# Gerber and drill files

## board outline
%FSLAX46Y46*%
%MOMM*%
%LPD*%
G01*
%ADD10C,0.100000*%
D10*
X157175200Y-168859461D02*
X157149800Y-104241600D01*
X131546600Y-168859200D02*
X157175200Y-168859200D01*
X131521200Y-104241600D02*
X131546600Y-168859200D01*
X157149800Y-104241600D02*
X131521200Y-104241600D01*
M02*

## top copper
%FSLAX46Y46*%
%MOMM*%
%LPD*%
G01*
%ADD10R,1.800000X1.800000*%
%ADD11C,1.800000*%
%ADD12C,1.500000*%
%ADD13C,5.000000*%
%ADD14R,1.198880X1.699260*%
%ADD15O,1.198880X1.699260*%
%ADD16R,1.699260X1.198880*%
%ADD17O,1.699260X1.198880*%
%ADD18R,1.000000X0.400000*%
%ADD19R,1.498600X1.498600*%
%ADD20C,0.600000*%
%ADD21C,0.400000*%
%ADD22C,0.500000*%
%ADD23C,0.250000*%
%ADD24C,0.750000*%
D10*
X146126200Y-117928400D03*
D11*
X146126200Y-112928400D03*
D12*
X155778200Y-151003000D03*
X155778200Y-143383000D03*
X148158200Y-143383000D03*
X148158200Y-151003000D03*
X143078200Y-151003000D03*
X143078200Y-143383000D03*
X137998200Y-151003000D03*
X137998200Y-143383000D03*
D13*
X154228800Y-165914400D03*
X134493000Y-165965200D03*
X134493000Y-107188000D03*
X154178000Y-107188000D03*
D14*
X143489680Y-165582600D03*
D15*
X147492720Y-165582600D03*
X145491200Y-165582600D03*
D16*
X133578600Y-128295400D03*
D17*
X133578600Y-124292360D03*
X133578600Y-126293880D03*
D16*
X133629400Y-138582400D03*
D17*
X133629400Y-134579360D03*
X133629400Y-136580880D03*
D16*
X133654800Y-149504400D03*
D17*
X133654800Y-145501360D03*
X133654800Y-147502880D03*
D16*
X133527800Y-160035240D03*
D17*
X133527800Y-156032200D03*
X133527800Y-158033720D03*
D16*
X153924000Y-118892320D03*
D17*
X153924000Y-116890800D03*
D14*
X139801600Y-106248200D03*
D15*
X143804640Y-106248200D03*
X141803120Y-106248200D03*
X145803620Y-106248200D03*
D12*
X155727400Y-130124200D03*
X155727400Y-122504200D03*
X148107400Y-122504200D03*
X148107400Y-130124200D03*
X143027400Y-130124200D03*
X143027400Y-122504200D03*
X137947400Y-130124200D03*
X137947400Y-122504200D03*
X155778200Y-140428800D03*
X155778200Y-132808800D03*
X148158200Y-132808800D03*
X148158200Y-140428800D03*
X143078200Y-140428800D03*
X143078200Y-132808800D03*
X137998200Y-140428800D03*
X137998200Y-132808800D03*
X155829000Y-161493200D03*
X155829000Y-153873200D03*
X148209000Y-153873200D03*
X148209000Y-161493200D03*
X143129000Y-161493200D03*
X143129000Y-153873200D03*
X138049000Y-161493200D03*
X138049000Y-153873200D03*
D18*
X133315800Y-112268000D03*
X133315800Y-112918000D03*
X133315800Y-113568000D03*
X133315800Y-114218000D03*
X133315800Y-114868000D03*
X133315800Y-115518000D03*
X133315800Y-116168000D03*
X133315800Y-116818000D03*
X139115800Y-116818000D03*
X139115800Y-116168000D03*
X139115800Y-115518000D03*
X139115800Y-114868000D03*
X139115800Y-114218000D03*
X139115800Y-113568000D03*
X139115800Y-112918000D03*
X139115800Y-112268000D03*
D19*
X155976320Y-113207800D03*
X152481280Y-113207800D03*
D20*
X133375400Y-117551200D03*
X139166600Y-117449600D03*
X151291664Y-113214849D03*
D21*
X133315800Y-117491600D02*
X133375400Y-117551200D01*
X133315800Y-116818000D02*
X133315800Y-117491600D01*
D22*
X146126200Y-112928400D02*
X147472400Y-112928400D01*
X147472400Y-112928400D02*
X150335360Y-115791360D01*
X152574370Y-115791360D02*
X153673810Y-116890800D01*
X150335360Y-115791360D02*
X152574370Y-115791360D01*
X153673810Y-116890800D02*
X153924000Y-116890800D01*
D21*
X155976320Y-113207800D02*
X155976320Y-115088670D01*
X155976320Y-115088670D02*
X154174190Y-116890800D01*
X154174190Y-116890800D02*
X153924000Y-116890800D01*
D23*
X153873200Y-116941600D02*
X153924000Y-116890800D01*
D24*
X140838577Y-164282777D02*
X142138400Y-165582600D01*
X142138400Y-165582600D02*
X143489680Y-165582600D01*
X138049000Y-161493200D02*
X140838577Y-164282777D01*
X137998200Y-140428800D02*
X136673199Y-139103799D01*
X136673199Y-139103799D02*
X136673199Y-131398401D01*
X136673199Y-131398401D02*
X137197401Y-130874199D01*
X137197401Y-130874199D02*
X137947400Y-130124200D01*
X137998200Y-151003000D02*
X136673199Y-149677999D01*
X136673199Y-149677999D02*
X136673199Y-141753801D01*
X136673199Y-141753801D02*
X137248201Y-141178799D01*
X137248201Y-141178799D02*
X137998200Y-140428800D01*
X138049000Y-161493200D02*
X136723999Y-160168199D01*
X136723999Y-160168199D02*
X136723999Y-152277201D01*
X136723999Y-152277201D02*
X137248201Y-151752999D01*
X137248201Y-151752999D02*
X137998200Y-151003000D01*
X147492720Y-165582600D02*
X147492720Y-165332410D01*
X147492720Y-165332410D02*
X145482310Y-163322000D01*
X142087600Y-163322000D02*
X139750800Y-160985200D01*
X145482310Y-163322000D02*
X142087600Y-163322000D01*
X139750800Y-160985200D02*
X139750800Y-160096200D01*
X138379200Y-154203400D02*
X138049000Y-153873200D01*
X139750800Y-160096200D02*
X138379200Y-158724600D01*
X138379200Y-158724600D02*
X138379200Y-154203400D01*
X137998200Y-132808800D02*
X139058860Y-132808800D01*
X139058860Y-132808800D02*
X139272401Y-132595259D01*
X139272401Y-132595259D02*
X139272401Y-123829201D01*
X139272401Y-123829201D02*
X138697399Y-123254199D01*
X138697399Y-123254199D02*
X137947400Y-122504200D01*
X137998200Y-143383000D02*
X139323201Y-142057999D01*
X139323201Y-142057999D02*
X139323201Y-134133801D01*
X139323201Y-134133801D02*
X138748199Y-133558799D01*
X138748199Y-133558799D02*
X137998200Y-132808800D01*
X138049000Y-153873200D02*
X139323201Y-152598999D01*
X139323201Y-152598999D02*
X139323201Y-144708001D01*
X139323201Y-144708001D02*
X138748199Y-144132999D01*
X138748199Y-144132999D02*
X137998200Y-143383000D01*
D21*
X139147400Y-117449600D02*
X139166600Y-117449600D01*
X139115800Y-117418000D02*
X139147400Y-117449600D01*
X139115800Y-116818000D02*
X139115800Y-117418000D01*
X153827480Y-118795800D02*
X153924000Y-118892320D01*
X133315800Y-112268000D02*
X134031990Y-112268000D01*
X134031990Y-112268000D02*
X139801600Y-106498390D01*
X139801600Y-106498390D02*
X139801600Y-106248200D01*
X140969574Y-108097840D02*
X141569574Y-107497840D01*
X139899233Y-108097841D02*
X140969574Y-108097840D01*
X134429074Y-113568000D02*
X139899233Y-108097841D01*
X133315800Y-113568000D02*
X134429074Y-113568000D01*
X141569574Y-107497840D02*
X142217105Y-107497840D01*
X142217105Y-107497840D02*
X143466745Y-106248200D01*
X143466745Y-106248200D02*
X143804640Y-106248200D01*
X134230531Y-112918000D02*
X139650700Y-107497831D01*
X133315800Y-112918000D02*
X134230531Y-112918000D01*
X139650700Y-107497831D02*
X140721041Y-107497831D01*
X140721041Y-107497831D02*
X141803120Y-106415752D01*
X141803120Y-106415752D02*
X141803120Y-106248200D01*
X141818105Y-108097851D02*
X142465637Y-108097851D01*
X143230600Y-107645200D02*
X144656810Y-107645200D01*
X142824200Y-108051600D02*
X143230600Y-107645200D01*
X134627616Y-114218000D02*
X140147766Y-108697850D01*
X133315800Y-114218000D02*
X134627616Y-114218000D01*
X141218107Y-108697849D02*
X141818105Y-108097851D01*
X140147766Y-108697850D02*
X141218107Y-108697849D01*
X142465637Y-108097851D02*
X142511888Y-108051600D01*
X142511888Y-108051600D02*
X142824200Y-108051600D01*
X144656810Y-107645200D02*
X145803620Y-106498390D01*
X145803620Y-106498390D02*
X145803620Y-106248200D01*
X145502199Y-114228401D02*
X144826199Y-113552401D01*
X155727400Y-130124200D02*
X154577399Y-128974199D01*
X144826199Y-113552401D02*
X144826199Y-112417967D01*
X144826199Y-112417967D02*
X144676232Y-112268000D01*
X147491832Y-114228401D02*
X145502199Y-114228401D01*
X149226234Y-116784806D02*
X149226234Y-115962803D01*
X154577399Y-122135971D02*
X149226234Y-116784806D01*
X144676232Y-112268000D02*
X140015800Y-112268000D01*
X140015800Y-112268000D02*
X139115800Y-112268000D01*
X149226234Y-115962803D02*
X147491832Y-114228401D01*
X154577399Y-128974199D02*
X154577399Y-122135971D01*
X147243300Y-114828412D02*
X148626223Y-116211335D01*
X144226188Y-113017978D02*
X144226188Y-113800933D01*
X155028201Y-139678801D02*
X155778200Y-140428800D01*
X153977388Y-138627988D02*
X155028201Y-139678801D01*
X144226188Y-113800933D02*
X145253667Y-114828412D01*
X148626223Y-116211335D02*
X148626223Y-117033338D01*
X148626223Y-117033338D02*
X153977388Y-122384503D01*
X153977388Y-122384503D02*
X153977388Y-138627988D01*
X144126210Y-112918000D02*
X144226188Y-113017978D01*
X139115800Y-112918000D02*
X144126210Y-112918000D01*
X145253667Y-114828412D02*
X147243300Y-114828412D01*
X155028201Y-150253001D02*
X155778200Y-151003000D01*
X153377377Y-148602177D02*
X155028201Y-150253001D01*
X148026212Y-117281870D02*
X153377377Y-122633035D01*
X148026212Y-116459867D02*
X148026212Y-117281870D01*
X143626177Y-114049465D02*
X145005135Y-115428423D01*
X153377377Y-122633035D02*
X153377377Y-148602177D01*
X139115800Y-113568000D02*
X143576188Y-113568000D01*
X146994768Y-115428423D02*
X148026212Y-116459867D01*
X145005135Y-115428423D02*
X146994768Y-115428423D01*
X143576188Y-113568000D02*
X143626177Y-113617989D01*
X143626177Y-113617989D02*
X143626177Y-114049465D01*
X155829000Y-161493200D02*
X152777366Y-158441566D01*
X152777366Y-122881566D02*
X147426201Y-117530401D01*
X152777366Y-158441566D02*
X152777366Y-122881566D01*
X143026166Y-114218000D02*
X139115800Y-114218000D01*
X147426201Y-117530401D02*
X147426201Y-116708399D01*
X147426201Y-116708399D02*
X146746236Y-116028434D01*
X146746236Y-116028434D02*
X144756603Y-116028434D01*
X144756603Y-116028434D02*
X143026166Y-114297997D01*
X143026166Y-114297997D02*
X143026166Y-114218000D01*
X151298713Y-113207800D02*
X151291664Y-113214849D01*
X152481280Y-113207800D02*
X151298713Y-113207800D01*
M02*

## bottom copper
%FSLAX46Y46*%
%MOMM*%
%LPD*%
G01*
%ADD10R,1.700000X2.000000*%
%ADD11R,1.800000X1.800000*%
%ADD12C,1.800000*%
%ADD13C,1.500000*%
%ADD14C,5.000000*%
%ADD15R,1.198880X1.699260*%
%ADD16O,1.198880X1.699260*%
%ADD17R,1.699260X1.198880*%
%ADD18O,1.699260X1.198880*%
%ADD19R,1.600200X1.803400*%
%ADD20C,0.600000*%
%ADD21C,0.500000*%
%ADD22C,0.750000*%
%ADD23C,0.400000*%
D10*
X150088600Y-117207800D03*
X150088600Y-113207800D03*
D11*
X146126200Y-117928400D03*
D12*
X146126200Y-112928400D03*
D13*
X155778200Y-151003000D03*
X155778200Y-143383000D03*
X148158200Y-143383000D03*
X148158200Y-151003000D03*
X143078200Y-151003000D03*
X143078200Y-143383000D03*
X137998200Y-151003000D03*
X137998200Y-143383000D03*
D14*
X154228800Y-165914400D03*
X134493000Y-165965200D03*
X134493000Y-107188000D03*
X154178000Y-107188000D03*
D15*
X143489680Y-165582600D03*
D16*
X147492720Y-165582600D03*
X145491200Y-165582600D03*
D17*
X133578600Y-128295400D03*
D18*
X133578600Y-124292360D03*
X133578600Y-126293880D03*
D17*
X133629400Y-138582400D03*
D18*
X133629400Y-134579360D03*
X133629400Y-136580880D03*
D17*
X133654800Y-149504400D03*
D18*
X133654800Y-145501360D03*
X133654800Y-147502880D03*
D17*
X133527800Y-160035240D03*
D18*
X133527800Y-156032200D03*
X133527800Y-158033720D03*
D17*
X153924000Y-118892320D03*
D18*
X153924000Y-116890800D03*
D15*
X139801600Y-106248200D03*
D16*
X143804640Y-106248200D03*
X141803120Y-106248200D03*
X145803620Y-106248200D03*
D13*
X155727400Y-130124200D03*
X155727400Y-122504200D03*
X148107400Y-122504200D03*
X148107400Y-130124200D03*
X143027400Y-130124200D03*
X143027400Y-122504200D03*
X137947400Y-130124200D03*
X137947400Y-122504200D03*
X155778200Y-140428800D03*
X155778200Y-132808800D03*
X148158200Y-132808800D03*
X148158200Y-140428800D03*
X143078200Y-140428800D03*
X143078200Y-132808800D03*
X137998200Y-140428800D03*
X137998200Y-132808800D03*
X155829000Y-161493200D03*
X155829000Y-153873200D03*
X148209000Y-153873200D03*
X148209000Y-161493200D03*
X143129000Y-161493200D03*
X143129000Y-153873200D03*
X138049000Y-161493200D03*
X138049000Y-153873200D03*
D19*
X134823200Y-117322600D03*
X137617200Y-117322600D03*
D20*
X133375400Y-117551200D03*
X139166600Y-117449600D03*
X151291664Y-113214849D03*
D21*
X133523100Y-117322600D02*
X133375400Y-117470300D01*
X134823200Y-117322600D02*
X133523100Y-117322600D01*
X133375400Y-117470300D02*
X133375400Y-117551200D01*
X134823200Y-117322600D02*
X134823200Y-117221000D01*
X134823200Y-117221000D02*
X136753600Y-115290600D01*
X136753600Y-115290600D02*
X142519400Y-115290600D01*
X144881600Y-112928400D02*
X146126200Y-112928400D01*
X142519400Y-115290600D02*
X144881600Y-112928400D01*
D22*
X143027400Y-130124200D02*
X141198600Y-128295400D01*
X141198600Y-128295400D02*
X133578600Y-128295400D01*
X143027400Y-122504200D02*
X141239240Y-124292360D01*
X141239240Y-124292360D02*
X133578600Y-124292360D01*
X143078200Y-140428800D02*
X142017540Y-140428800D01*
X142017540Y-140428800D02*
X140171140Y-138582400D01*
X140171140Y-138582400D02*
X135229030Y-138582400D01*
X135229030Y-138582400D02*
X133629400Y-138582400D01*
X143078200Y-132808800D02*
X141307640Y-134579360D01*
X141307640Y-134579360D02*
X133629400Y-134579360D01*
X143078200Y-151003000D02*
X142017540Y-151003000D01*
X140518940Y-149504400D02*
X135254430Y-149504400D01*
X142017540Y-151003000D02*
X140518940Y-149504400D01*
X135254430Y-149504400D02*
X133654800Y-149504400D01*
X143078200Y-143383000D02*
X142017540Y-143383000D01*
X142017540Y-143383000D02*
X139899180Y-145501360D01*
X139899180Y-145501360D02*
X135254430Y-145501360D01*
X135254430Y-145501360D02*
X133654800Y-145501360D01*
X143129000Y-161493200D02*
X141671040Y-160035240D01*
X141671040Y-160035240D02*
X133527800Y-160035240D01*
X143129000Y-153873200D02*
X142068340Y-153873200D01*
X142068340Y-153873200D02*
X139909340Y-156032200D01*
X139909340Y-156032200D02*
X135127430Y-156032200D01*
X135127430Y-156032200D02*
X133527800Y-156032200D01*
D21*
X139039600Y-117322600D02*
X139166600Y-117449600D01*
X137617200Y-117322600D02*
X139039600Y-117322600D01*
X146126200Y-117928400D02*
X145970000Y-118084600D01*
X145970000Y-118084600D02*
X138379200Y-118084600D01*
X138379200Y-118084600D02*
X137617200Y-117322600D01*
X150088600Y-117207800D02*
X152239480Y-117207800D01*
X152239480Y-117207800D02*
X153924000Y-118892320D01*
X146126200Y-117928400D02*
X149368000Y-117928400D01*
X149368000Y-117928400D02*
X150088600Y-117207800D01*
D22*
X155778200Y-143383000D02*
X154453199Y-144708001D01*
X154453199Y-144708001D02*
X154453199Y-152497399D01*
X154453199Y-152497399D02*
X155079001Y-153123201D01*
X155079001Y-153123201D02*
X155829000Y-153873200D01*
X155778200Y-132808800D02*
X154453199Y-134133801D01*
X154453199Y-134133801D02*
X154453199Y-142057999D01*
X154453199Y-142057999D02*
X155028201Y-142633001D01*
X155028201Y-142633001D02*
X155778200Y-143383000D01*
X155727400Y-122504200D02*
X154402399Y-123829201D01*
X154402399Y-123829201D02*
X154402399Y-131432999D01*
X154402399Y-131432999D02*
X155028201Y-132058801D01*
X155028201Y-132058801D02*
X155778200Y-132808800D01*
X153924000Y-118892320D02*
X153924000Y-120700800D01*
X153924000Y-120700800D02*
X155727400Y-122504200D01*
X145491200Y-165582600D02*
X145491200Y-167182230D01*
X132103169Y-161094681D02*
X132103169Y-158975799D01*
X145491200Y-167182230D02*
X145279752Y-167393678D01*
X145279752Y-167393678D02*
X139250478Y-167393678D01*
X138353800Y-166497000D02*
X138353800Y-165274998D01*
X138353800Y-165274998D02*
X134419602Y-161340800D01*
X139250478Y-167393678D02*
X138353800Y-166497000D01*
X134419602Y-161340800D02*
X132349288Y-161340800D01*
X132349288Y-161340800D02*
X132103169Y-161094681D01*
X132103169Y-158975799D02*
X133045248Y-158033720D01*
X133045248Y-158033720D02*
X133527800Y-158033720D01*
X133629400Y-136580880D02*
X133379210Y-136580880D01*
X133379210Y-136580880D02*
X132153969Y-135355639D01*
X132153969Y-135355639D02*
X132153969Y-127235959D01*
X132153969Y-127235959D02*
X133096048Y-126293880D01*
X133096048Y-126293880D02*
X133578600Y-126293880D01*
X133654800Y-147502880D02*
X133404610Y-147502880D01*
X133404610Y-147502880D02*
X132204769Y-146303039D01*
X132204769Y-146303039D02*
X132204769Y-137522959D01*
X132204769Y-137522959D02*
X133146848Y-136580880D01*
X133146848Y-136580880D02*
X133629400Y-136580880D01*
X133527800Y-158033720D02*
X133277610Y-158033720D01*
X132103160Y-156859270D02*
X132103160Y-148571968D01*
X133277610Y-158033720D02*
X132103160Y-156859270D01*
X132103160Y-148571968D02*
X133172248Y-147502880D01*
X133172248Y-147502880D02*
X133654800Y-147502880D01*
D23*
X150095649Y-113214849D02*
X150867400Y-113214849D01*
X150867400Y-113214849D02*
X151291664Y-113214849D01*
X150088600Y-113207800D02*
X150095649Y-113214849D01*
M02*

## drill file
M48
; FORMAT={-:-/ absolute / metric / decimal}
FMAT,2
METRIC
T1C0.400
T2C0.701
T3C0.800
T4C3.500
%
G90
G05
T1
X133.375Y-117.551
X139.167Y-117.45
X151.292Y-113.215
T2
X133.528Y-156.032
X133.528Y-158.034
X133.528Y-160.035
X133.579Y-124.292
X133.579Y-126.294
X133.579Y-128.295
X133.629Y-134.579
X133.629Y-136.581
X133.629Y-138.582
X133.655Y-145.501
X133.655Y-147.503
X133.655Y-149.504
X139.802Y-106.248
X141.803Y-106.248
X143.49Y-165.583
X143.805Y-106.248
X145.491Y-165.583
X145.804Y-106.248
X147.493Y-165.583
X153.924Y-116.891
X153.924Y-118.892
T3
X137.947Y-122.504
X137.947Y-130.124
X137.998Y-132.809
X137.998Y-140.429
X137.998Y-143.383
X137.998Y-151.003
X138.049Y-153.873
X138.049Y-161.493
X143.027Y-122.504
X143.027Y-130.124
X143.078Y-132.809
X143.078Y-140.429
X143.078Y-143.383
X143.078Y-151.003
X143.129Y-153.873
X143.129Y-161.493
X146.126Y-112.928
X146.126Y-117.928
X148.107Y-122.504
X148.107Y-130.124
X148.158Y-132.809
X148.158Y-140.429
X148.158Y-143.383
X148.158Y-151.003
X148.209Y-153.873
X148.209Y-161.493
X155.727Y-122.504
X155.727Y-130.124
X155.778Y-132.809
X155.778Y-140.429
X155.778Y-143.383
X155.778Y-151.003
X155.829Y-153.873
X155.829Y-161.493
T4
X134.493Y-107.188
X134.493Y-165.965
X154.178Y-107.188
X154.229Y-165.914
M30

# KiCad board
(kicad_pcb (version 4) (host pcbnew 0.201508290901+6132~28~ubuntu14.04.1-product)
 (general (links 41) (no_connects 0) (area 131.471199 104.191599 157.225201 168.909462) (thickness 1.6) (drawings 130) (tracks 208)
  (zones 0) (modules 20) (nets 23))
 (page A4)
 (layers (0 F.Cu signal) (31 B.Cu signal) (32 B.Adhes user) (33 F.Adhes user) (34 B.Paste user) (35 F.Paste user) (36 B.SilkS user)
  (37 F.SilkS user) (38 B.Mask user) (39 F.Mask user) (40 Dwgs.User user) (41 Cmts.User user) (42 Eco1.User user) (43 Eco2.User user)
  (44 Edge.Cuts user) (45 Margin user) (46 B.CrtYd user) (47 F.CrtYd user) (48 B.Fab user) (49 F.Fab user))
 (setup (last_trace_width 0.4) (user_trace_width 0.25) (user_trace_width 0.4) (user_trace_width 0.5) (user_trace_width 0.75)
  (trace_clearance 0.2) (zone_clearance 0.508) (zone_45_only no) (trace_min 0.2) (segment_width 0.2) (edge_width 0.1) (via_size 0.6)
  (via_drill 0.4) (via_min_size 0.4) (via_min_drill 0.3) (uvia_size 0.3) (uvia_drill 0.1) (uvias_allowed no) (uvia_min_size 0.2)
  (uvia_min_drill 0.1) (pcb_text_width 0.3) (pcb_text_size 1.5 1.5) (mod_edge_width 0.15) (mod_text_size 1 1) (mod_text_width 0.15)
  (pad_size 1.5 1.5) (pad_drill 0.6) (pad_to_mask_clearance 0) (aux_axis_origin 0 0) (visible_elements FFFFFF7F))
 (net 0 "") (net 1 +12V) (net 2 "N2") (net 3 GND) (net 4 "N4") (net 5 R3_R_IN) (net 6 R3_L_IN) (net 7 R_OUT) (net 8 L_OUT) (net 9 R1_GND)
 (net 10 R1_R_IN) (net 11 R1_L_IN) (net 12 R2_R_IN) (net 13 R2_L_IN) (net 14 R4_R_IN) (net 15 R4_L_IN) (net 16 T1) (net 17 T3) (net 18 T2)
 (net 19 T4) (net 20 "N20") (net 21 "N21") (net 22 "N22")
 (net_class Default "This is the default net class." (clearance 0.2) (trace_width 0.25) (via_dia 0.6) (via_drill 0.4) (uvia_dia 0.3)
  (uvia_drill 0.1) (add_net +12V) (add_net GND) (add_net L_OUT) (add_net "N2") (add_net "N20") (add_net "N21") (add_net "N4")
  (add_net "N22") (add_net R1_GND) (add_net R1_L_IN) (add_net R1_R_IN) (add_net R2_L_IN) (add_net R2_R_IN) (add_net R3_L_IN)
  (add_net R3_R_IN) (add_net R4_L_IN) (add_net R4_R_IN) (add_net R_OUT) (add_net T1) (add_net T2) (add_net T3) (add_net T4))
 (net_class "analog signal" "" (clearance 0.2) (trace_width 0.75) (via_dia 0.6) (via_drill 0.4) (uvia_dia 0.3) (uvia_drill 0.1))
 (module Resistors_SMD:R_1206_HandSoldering (layer B.Cu) (at 150.0886 115.2078 90)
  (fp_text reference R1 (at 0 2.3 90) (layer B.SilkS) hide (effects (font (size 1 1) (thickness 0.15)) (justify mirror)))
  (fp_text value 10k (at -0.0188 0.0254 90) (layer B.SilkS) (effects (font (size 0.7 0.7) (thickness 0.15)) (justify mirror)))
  (pad 1 smd rect (at -2 0 90) (size 2 1.7) (layers B.Cu B.Paste B.Mask) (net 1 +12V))
  (pad 2 smd rect (at 2 0 90) (size 2 1.7) (layers B.Cu B.Paste B.Mask) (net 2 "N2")))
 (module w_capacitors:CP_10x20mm (layer F.Cu) (at 146.1262 115.4284)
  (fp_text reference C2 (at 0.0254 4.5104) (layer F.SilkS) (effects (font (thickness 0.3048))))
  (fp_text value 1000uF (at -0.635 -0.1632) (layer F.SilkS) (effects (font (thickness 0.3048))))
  (pad 1 thru_hole rect (at 0 2.5) (size 1.8 1.8) (drill 0.8) (layers *.Cu *.Mask F.SilkS) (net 1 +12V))
  (pad 2 thru_hole circle (at 0 -2.5) (size 1.8 1.8) (drill 0.8) (layers *.Cu *.Mask F.SilkS) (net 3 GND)))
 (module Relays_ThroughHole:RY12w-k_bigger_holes (layer F.Cu) (at 156.9782 152.103 180)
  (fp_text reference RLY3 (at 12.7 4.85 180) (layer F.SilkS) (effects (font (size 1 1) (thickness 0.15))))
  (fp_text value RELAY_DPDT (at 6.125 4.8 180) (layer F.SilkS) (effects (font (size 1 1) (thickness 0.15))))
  (pad 1 thru_hole circle (at 1.2 1.1 180) (size 1.5 1.5) (drill 0.8) (layers *.Cu *.Mask F.SilkS) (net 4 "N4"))
  (pad 8 thru_hole circle (at 1.2 8.72 180) (size 1.5 1.5) (drill 0.8) (layers *.Cu *.Mask F.SilkS) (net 1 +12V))
  (pad 7 thru_hole circle (at 8.82 8.72 180) (size 1.5 1.5) (drill 0.8) (layers *.Cu *.Mask F.SilkS))
  (pad 2 thru_hole circle (at 8.82 1.1 180) (size 1.5 1.5) (drill 0.8) (layers *.Cu *.Mask F.SilkS))
  (pad 3 thru_hole circle (at 13.9 1.1 180) (size 1.5 1.5) (drill 0.8) (layers *.Cu *.Mask F.SilkS) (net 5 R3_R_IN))
  (pad 6 thru_hole circle (at 13.9 8.72 180) (size 1.5 1.5) (drill 0.8) (layers *.Cu *.Mask F.SilkS) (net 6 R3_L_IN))
  (pad 4 thru_hole circle (at 18.98 1.1 180) (size 1.5 1.5) (drill 0.8) (layers *.Cu *.Mask F.SilkS) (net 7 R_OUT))
  (pad 5 thru_hole circle (at 18.98 8.72 180) (size 1.5 1.5) (drill 0.8) (layers *.Cu *.Mask F.SilkS) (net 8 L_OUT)))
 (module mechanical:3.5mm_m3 (layer F.Cu) (at 154.2288 166.0144)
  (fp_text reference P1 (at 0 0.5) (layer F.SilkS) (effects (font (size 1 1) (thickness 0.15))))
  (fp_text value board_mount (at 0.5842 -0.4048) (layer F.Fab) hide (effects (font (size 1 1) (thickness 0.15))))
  (pad 1 thru_hole circle (at 0 -0.1) (size 5 5) (drill 3.5) (layers *.Cu *.Mask F.SilkS)))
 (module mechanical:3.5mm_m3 (layer F.Cu) (at 134.493 166.0652)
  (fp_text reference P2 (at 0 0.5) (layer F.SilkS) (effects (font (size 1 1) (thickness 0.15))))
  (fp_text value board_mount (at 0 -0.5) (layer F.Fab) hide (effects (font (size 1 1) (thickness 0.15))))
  (pad 1 thru_hole circle (at 0 -0.1) (size 5 5) (drill 3.5) (layers *.Cu *.Mask F.SilkS)))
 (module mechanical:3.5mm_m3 (layer F.Cu) (at 134.493 107.288)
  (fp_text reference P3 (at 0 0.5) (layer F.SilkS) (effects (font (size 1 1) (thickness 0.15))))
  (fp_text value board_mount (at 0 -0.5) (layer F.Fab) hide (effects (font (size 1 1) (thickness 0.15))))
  (pad 1 thru_hole circle (at 0 -0.1) (size 5 5) (drill 3.5) (layers *.Cu *.Mask F.SilkS)))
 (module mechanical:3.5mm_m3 (layer F.Cu) (at 154.178 107.288)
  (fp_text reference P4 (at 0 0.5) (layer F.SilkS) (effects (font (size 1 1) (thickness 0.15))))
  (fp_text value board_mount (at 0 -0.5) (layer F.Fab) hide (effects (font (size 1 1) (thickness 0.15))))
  (pad 1 thru_hole circle (at 0 -0.1) (size 5 5) (drill 3.5) (layers *.Cu *.Mask F.SilkS)))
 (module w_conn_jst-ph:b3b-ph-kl (layer F.Cu) (at 145.4912 165.5826)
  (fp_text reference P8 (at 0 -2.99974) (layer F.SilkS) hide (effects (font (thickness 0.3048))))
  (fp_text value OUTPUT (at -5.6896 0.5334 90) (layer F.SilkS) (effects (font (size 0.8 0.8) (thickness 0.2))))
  (pad 1 thru_hole rect (at -2.00152 0) (size 1.19888 1.69926) (drill 0.70104) (layers *.Cu *.Mask F.SilkS) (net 7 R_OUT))
  (pad 3 thru_hole oval (at 2.00152 0) (size 1.19888 1.69926) (drill 0.70104) (layers *.Cu *.Mask F.SilkS) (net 8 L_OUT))
  (pad 2 thru_hole oval (at 0 0) (size 1.19888 1.69926) (drill 0.70104) (layers *.Cu *.Mask F.SilkS) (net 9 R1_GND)))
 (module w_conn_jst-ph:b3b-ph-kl (layer F.Cu) (at 133.5786 126.29388 90)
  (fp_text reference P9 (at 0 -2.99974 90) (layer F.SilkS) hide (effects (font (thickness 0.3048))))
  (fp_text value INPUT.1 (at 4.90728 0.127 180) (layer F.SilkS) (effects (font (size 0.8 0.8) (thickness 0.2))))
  (pad 1 thru_hole rect (at -2.00152 0 90) (size 1.19888 1.69926) (drill 0.70104) (layers *.Cu *.Mask F.SilkS) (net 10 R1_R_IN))
  (pad 3 thru_hole oval (at 2.00152 0 90) (size 1.19888 1.69926) (drill 0.70104) (layers *.Cu *.Mask F.SilkS) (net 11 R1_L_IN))
  (pad 2 thru_hole oval (at 0 0 90) (size 1.19888 1.69926) (drill 0.70104) (layers *.Cu *.Mask F.SilkS) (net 9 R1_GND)))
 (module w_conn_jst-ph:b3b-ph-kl (layer F.Cu) (at 133.6294 136.58088 90)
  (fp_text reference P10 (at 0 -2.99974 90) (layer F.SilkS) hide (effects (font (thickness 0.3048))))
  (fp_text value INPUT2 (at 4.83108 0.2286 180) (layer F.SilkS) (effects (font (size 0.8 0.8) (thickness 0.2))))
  (pad 1 thru_hole rect (at -2.00152 0 90) (size 1.19888 1.69926) (drill 0.70104) (layers *.Cu *.Mask F.SilkS) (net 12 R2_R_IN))
  (pad 3 thru_hole oval (at 2.00152 0 90) (size 1.19888 1.69926) (drill 0.70104) (layers *.Cu *.Mask F.SilkS) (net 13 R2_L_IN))
  (pad 2 thru_hole oval (at 0 0 90) (size 1.19888 1.69926) (drill 0.70104) (layers *.Cu *.Mask F.SilkS) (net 9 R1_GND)))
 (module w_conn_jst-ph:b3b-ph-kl (layer F.Cu) (at 133.6548 147.50288 90)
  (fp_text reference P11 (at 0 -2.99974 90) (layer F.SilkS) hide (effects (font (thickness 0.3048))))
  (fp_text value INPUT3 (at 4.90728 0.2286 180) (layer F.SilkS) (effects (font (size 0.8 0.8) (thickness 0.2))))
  (pad 1 thru_hole rect (at -2.00152 0 90) (size 1.19888 1.69926) (drill 0.70104) (layers *.Cu *.Mask F.SilkS) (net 5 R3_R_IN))
  (pad 3 thru_hole oval (at 2.00152 0 90) (size 1.19888 1.69926) (drill 0.70104) (layers *.Cu *.Mask F.SilkS) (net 6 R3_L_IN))
  (pad 2 thru_hole oval (at 0 0 90) (size 1.19888 1.69926) (drill 0.70104) (layers *.Cu *.Mask F.SilkS) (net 9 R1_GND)))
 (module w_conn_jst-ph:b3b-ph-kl (layer F.Cu) (at 133.5278 158.03372 90)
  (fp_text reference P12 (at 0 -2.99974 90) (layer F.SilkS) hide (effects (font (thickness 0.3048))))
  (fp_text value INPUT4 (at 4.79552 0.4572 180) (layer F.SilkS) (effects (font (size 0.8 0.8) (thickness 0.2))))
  (pad 1 thru_hole rect (at -2.00152 0 90) (size 1.19888 1.69926) (drill 0.70104) (layers *.Cu *.Mask F.SilkS) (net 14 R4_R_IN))
  (pad 3 thru_hole oval (at 2.00152 0 90) (size 1.19888 1.69926) (drill 0.70104) (layers *.Cu *.Mask F.SilkS) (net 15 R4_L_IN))
  (pad 2 thru_hole oval (at 0 0 90) (size 1.19888 1.69926) (drill 0.70104) (layers *.Cu *.Mask F.SilkS) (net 9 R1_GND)))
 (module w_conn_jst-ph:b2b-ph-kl (layer F.Cu) (at 153.924 117.89156 90)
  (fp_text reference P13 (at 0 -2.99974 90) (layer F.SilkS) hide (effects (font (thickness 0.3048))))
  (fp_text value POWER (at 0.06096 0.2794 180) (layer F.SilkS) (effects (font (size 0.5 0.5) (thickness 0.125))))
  (pad 1 thru_hole rect (at -1.00076 0 90) (size 1.19888 1.69926) (drill 0.70104) (layers *.Cu *.Mask F.SilkS) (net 1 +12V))
  (pad 2 thru_hole oval (at 1.00076 0 90) (size 1.19888 1.69926) (drill 0.70104) (layers *.Cu *.Mask F.SilkS) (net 3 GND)))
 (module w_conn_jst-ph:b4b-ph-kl (layer F.Cu) (at 142.80388 106.2482)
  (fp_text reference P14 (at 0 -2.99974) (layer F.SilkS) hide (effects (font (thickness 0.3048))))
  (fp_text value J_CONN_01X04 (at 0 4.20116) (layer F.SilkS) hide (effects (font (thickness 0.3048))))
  (pad 1 thru_hole rect (at -3.00228 0) (size 1.19888 1.69926) (drill 0.70104) (layers *.Cu *.Mask F.SilkS) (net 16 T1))
  (pad 3 thru_hole oval (at 1.00076 0) (size 1.19888 1.69926) (drill 0.70104) (layers *.Cu *.Mask F.SilkS) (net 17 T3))
  (pad 2 thru_hole oval (at -1.00076 0) (size 1.19888 1.69926) (drill 0.70104) (layers *.Cu *.Mask F.SilkS) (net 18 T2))
  (pad 4 thru_hole oval (at 2.99974 0) (size 1.19888 1.69926) (drill 0.70104) (layers *.Cu *.Mask F.SilkS) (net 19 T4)))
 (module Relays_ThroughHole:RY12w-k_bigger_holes (layer F.Cu) (at 156.9274 131.2242 180)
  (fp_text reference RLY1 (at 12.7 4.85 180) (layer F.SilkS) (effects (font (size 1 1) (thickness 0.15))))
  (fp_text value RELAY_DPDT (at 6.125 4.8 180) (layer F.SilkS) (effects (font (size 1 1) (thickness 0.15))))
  (pad 1 thru_hole circle (at 1.2 1.1 180) (size 1.5 1.5) (drill 0.8) (layers *.Cu *.Mask F.SilkS) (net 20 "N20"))
  (pad 8 thru_hole circle (at 1.2 8.72 180) (size 1.5 1.5) (drill 0.8) (layers *.Cu *.Mask F.SilkS) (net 1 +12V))
  (pad 7 thru_hole circle (at 8.82 8.72 180) (size 1.5 1.5) (drill 0.8) (layers *.Cu *.Mask F.SilkS))
  (pad 2 thru_hole circle (at 8.82 1.1 180) (size 1.5 1.5) (drill 0.8) (layers *.Cu *.Mask F.SilkS))
  (pad 3 thru_hole circle (at 13.9 1.1 180) (size 1.5 1.5) (drill 0.8) (layers *.Cu *.Mask F.SilkS) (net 10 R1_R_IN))
  (pad 6 thru_hole circle (at 13.9 8.72 180) (size 1.5 1.5) (drill 0.8) (layers *.Cu *.Mask F.SilkS) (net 11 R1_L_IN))
  (pad 4 thru_hole circle (at 18.98 1.1 180) (size 1.5 1.5) (drill 0.8) (layers *.Cu *.Mask F.SilkS) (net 7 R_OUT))
  (pad 5 thru_hole circle (at 18.98 8.72 180) (size 1.5 1.5) (drill 0.8) (layers *.Cu *.Mask F.SilkS) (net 8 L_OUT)))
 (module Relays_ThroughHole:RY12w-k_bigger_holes (layer F.Cu) (at 156.9782 141.5288 180)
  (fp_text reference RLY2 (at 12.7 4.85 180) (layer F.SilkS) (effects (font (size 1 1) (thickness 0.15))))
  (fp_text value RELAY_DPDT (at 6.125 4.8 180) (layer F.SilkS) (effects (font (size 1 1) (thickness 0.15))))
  (pad 1 thru_hole circle (at 1.2 1.1 180) (size 1.5 1.5) (drill 0.8) (layers *.Cu *.Mask F.SilkS) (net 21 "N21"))
  (pad 8 thru_hole circle (at 1.2 8.72 180) (size 1.5 1.5) (drill 0.8) (layers *.Cu *.Mask F.SilkS) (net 1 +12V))
  (pad 7 thru_hole circle (at 8.82 8.72 180) (size 1.5 1.5) (drill 0.8) (layers *.Cu *.Mask F.SilkS))
  (pad 2 thru_hole circle (at 8.82 1.1 180) (size 1.5 1.5) (drill 0.8) (layers *.Cu *.Mask F.SilkS))
  (pad 3 thru_hole circle (at 13.9 1.1 180) (size 1.5 1.5) (drill 0.8) (layers *.Cu *.Mask F.SilkS) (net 12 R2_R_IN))
  (pad 6 thru_hole circle (at 13.9 8.72 180) (size 1.5 1.5) (drill 0.8) (layers *.Cu *.Mask F.SilkS) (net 13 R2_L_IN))
  (pad 4 thru_hole circle (at 18.98 1.1 180) (size 1.5 1.5) (drill 0.8) (layers *.Cu *.Mask F.SilkS) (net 7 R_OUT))
  (pad 5 thru_hole circle (at 18.98 8.72 180) (size 1.5 1.5) (drill 0.8) (layers *.Cu *.Mask F.SilkS) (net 8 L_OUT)))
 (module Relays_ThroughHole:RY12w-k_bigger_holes (layer F.Cu) (at 157.029 162.5932 180)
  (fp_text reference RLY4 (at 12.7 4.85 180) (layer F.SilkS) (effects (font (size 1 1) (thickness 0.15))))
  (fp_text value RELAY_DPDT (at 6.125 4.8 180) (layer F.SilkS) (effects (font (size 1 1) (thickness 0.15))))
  (pad 1 thru_hole circle (at 1.2 1.1 180) (size 1.5 1.5) (drill 0.8) (layers *.Cu *.Mask F.SilkS) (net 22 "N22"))
  (pad 8 thru_hole circle (at 1.2 8.72 180) (size 1.5 1.5) (drill 0.8) (layers *.Cu *.Mask F.SilkS) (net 1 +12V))
  (pad 7 thru_hole circle (at 8.82 8.72 180) (size 1.5 1.5) (drill 0.8) (layers *.Cu *.Mask F.SilkS))
  (pad 2 thru_hole circle (at 8.82 1.1 180) (size 1.5 1.5) (drill 0.8) (layers *.Cu *.Mask F.SilkS))
  (pad 3 thru_hole circle (at 13.9 1.1 180) (size 1.5 1.5) (drill 0.8) (layers *.Cu *.Mask F.SilkS) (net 14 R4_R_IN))
  (pad 6 thru_hole circle (at 13.9 8.72 180) (size 1.5 1.5) (drill 0.8) (layers *.Cu *.Mask F.SilkS) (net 15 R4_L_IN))
  (pad 4 thru_hole circle (at 18.98 1.1 180) (size 1.5 1.5) (drill 0.8) (layers *.Cu *.Mask F.SilkS) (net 7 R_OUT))
  (pad 5 thru_hole circle (at 18.98 8.72 180) (size 1.5 1.5) (drill 0.8) (layers *.Cu *.Mask F.SilkS) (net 8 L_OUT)))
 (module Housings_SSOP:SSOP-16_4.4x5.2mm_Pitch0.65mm (layer F.Cu) (at 136.2158 114.543)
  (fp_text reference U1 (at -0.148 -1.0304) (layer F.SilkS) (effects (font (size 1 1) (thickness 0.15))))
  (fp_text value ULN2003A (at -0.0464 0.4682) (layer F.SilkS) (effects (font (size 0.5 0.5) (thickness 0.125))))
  (pad 1 smd rect (at -2.9 -2.275) (size 1 0.4) (layers F.Cu F.Paste F.Mask) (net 16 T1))
  (pad 2 smd rect (at -2.9 -1.625) (size 1 0.4) (layers F.Cu F.Paste F.Mask) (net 18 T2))
  (pad 3 smd rect (at -2.9 -0.975) (size 1 0.4) (layers F.Cu F.Paste F.Mask) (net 17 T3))
  (pad 4 smd rect (at -2.9 -0.325) (size 1 0.4) (layers F.Cu F.Paste F.Mask) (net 19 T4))
  (pad 5 smd rect (at -2.9 0.325) (size 1 0.4) (layers F.Cu F.Paste F.Mask))
  (pad 6 smd rect (at -2.9 0.975) (size 1 0.4) (layers F.Cu F.Paste F.Mask))
  (pad 7 smd rect (at -2.9 1.625) (size 1 0.4) (layers F.Cu F.Paste F.Mask))
  (pad 8 smd rect (at -2.9 2.275) (size 1 0.4) (layers F.Cu F.Paste F.Mask) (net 3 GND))
  (pad 9 smd rect (at 2.9 2.275) (size 1 0.4) (layers F.Cu F.Paste F.Mask) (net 1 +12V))
  (pad 10 smd rect (at 2.9 1.625) (size 1 0.4) (layers F.Cu F.Paste F.Mask))
  (pad 11 smd rect (at 2.9 0.975) (size 1 0.4) (layers F.Cu F.Paste F.Mask))
  (pad 12 smd rect (at 2.9 0.325) (size 1 0.4) (layers F.Cu F.Paste F.Mask))
  (pad 13 smd rect (at 2.9 -0.325) (size 1 0.4) (layers F.Cu F.Paste F.Mask) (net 22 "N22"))
  (pad 14 smd rect (at 2.9 -0.975) (size 1 0.4) (layers F.Cu F.Paste F.Mask) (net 4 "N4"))
  (pad 15 smd rect (at 2.9 -1.625) (size 1 0.4) (layers F.Cu F.Paste F.Mask) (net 21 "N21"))
  (pad 16 smd rect (at 2.9 -2.275) (size 1 0.4) (layers F.Cu F.Paste F.Mask) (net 20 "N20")))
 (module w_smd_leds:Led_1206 (layer F.Cu) (at 154.2288 113.2078 180)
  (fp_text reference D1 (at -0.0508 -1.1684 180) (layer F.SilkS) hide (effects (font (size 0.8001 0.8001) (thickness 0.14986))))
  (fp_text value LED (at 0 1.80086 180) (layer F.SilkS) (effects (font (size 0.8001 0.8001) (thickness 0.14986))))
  (pad 1 smd rect (at -1.74752 0 180) (size 1.4986 1.4986) (layers F.Cu F.Paste F.Mask) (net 3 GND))
  (pad 2 smd rect (at 1.74752 0 180) (size 1.4986 1.4986) (layers F.Cu F.Paste F.Mask) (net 2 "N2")))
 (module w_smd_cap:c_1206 (layer B.Cu) (at 136.2202 117.3226 180)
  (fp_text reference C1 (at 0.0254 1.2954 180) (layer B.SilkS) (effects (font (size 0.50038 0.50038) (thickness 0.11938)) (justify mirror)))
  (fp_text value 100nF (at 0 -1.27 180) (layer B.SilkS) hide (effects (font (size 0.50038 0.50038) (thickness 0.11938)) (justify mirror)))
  (pad 1 smd rect (at 1.397 0 180) (size 1.6002 1.8034) (layers B.Cu B.Paste B.Mask) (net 3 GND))
  (pad 2 smd rect (at -1.397 0 180) (size 1.6002 1.8034) (layers B.Cu B.Paste B.Mask) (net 1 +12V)))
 (gr_line (start 157.1752 168.859461) (end 157.1498 104.2416) (layer Edge.Cuts) (width 0.1))
 (gr_line (start 131.5466 168.8592) (end 157.1752 168.8592) (layer Edge.Cuts) (width 0.1))
 (gr_line (start 131.5212 104.2416) (end 131.5466 168.8592) (layer Edge.Cuts) (width 0.1))
 (gr_line (start 157.1498 104.2416) (end 131.5212 104.2416) (layer Edge.Cuts) (width 0.1))
 (segment (start 133.3158 117.4916) (end 133.3754 117.5512) (width 0.4) (layer F.Cu) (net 3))
 (segment (start 133.3158 116.818) (end 133.3158 117.4916) (width 0.4) (layer F.Cu) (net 3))
 (segment (start 133.5231 117.3226) (end 133.3754 117.4703) (width 0.5) (layer B.Cu) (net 3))
 (segment (start 134.8232 117.3226) (end 133.5231 117.3226) (width 0.5) (layer B.Cu) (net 3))
 (segment (start 133.3754 117.4703) (end 133.3754 117.5512) (width 0.5) (layer B.Cu) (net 3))
 (via (at 133.3754 117.5512) (size 0.6) (drill 0.4) (layers F.Cu B.Cu) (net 3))
 (segment (start 134.8232 117.3226) (end 134.8232 117.221) (width 0.5) (layer B.Cu) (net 3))
 (segment (start 134.8232 117.221) (end 136.7536 115.2906) (width 0.5) (layer B.Cu) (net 3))
 (segment (start 136.7536 115.2906) (end 142.5194 115.2906) (width 0.5) (layer B.Cu) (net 3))
 (segment (start 144.8816 112.9284) (end 146.1262 112.9284) (width 0.5) (layer B.Cu) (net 3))
 (segment (start 142.5194 115.2906) (end 144.8816 112.9284) (width 0.5) (layer B.Cu) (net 3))
 (segment (start 146.1262 112.9284) (end 147.4724 112.9284) (width 0.5) (layer F.Cu) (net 3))
 (segment (start 147.4724 112.9284) (end 150.33536 115.79136) (width 0.5) (layer F.Cu) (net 3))
 (segment (start 152.57437 115.79136) (end 153.67381 116.8908) (width 0.5) (layer F.Cu) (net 3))
 (segment (start 150.33536 115.79136) (end 152.57437 115.79136) (width 0.5) (layer F.Cu) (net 3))
 (segment (start 153.67381 116.8908) (end 153.924 116.8908) (width 0.5) (layer F.Cu) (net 3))
 (segment (start 155.97632 113.2078) (end 155.97632 115.08867) (width 0.4) (layer F.Cu) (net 3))
 (segment (start 155.97632 115.08867) (end 154.17419 116.8908) (width 0.4) (layer F.Cu) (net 3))
 (segment (start 154.17419 116.8908) (end 153.924 116.8908) (width 0.4) (layer F.Cu) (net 3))
 (segment (start 153.8732 116.9416) (end 153.924 116.8908) (width 0.25) (layer F.Cu) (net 3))
 (segment (start 140.838577 164.282777) (end 142.1384 165.5826) (width 0.75) (layer F.Cu) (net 7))
 (segment (start 142.1384 165.5826) (end 143.48968 165.5826) (width 0.75) (layer F.Cu) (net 7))
 (segment (start 138.049 161.4932) (end 140.838577 164.282777) (width 0.75) (layer F.Cu) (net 7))
 (segment (start 137.9982 140.4288) (end 136.673199 139.103799) (width 0.75) (layer F.Cu) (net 7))
 (segment (start 136.673199 139.103799) (end 136.673199 131.398401) (width 0.75) (layer F.Cu) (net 7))
 (segment (start 136.673199 131.398401) (end 137.197401 130.874199) (width 0.75) (layer F.Cu) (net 7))
 (segment (start 137.197401 130.874199) (end 137.9474 130.1242) (width 0.75) (layer F.Cu) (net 7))
 (segment (start 137.9982 151.003) (end 136.673199 149.677999) (width 0.75) (layer F.Cu) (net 7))
 (segment (start 136.673199 149.677999) (end 136.673199 141.753801) (width 0.75) (layer F.Cu) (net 7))
 (segment (start 136.673199 141.753801) (end 137.248201 141.178799) (width 0.75) (layer F.Cu) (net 7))
 (segment (start 137.248201 141.178799) (end 137.9982 140.4288) (width 0.75) (layer F.Cu) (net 7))
 (segment (start 138.049 161.4932) (end 136.723999 160.168199) (width 0.75) (layer F.Cu) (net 7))
 (segment (start 136.723999 160.168199) (end 136.723999 152.277201) (width 0.75) (layer F.Cu) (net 7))
 (segment (start 136.723999 152.277201) (end 137.248201 151.752999) (width 0.75) (layer F.Cu) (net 7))
 (segment (start 137.248201 151.752999) (end 137.9982 151.003) (width 0.75) (layer F.Cu) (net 7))
 (segment (start 147.49272 165.5826) (end 147.49272 165.33241) (width 0.75) (layer F.Cu) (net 8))
 (segment (start 147.49272 165.33241) (end 145.48231 163.322) (width 0.75) (layer F.Cu) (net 8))
 (segment (start 142.0876 163.322) (end 139.7508 160.9852) (width 0.75) (layer F.Cu) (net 8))
 (segment (start 145.48231 163.322) (end 142.0876 163.322) (width 0.75) (layer F.Cu) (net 8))
 (segment (start 139.7508 160.9852) (end 139.7508 160.0962) (width 0.75) (layer F.Cu) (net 8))
 (segment (start 138.3792 154.2034) (end 138.049 153.8732) (width 0.75) (layer F.Cu) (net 8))
 (segment (start 139.7508 160.0962) (end 138.3792 158.7246) (width 0.75) (layer F.Cu) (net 8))
 (segment (start 138.3792 158.7246) (end 138.3792 154.2034) (width 0.75) (layer F.Cu) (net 8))
 (segment (start 137.9982 132.8088) (end 139.05886 132.8088) (width 0.75) (layer F.Cu) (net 8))
 (segment (start 139.05886 132.8088) (end 139.272401 132.595259) (width 0.75) (layer F.Cu) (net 8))
 (segment (start 139.272401 132.595259) (end 139.272401 123.829201) (width 0.75) (layer F.Cu) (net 8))
 (segment (start 139.272401 123.829201) (end 138.697399 123.254199) (width 0.75) (layer F.Cu) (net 8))
 (segment (start 138.697399 123.254199) (end 137.9474 122.5042) (width 0.75) (layer F.Cu) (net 8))
 (segment (start 137.9982 143.383) (end 139.323201 142.057999) (width 0.75) (layer F.Cu) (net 8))
 (segment (start 139.323201 142.057999) (end 139.323201 134.133801) (width 0.75) (layer F.Cu) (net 8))
 (segment (start 139.323201 134.133801) (end 138.748199 133.558799) (width 0.75) (layer F.Cu) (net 8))
 (segment (start 138.748199 133.558799) (end 137.9982 132.8088) (width 0.75) (layer F.Cu) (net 8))
 (segment (start 138.049 153.8732) (end 139.323201 152.598999) (width 0.75) (layer F.Cu) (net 8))
 (segment (start 139.323201 152.598999) (end 139.323201 144.708001) (width 0.75) (layer F.Cu) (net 8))
 (segment (start 139.323201 144.708001) (end 138.748199 144.132999) (width 0.75) (layer F.Cu) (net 8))
 (segment (start 138.748199 144.132999) (end 137.9982 143.383) (width 0.75) (layer F.Cu) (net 8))
 (segment (start 143.0274 130.1242) (end 141.1986 128.2954) (width 0.75) (layer B.Cu) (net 10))
 (segment (start 141.1986 128.2954) (end 133.5786 128.2954) (width 0.75) (layer B.Cu) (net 10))
 (segment (start 143.0274 122.5042) (end 141.23924 124.29236) (width 0.75) (layer B.Cu) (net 11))
 (segment (start 141.23924 124.29236) (end 133.5786 124.29236) (width 0.75) (layer B.Cu) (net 11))
 (segment (start 143.0782 140.4288) (end 142.01754 140.4288) (width 0.75) (layer B.Cu) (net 12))
 (segment (start 142.01754 140.4288) (end 140.17114 138.5824) (width 0.75) (layer B.Cu) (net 12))
 (segment (start 140.17114 138.5824) (end 135.22903 138.5824) (width 0.75) (layer B.Cu) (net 12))
 (segment (start 135.22903 138.5824) (end 133.6294 138.5824) (width 0.75) (layer B.Cu) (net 12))
 (segment (start 143.0782 132.8088) (end 141.30764 134.57936) (width 0.75) (layer B.Cu) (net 13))
 (segment (start 141.30764 134.57936) (end 133.6294 134.57936) (width 0.75) (layer B.Cu) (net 13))
 (segment (start 143.0782 151.003) (end 142.01754 151.003) (width 0.75) (layer B.Cu) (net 5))
 (segment (start 140.51894 149.5044) (end 135.25443 149.5044) (width 0.75) (layer B.Cu) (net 5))
 (segment (start 142.01754 151.003) (end 140.51894 149.5044) (width 0.75) (layer B.Cu) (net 5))
 (segment (start 135.25443 149.5044) (end 133.6548 149.5044) (width 0.75) (layer B.Cu) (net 5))
 (segment (start 143.0782 143.383) (end 142.01754 143.383) (width 0.75) (layer B.Cu) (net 6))
 (segment (start 142.01754 143.383) (end 139.89918 145.50136) (width 0.75) (layer B.Cu) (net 6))
 (segment (start 139.89918 145.50136) (end 135.25443 145.50136) (width 0.75) (layer B.Cu) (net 6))
 (segment (start 135.25443 145.50136) (end 133.6548 145.50136) (width 0.75) (layer B.Cu) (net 6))
 (segment (start 143.129 161.4932) (end 141.67104 160.03524) (width 0.75) (layer B.Cu) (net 14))
 (segment (start 141.67104 160.03524) (end 133.5278 160.03524) (width 0.75) (layer B.Cu) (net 14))
 (segment (start 143.129 153.8732) (end 142.06834 153.8732) (width 0.75) (layer B.Cu) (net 15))
 (segment (start 142.06834 153.8732) (end 139.90934 156.0322) (width 0.75) (layer B.Cu) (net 15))
 (segment (start 139.90934 156.0322) (end 135.12743 156.0322) (width 0.75) (layer B.Cu) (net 15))
 (segment (start 135.12743 156.0322) (end 133.5278 156.0322) (width 0.75) (layer B.Cu) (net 15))
 (segment (start 139.0396 117.3226) (end 139.1666 117.4496) (width 0.5) (layer B.Cu) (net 1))
 (segment (start 137.6172 117.3226) (end 139.0396 117.3226) (width 0.5) (layer B.Cu) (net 1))
 (segment (start 139.1474 117.4496) (end 139.1666 117.4496) (width 0.4) (layer F.Cu) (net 1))
 (segment (start 139.1158 117.418) (end 139.1474 117.4496) (width 0.4) (layer F.Cu) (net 1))
 (segment (start 139.1158 116.818) (end 139.1158 117.418) (width 0.4) (layer F.Cu) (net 1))
 (via (at 139.1666 117.4496) (size 0.6) (drill 0.4) (layers F.Cu B.Cu) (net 1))
 (segment (start 146.1262 117.9284) (end 145.97 118.0846) (width 0.5) (layer B.Cu) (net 1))
 (segment (start 145.97 118.0846) (end 138.3792 118.0846) (width 0.5) (layer B.Cu) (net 1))
 (segment (start 138.3792 118.0846) (end 137.6172 117.3226) (width 0.5) (layer B.Cu) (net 1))
 (segment (start 150.0886 117.2078) (end 152.23948 117.2078) (width 0.5) (layer B.Cu) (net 1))
 (segment (start 152.23948 117.2078) (end 153.924 118.89232) (width 0.5) (layer B.Cu) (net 1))
 (segment (start 146.1262 117.9284) (end 149.368 117.9284) (width 0.5) (layer B.Cu) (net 1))
 (segment (start 149.368 117.9284) (end 150.0886 117.2078) (width 0.5) (layer B.Cu) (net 1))
 (segment (start 155.7782 143.383) (end 154.453199 144.708001) (width 0.75) (layer B.Cu) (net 1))
 (segment (start 154.453199 144.708001) (end 154.453199 152.497399) (width 0.75) (layer B.Cu) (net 1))
 (segment (start 154.453199 152.497399) (end 155.079001 153.123201) (width 0.75) (layer B.Cu) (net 1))
 (segment (start 155.079001 153.123201) (end 155.829 153.8732) (width 0.75) (layer B.Cu) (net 1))
 (segment (start 155.7782 132.8088) (end 154.453199 134.133801) (width 0.75) (layer B.Cu) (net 1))
 (segment (start 154.453199 134.133801) (end 154.453199 142.057999) (width 0.75) (layer B.Cu) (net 1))
 (segment (start 154.453199 142.057999) (end 155.028201 142.633001) (width 0.75) (layer B.Cu) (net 1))
 (segment (start 155.028201 142.633001) (end 155.7782 143.383) (width 0.75) (layer B.Cu) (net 1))
 (segment (start 155.7274 122.5042) (end 154.402399 123.829201) (width 0.75) (layer B.Cu) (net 1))
 (segment (start 154.402399 123.829201) (end 154.402399 131.432999) (width 0.75) (layer B.Cu) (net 1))
 (segment (start 154.402399 131.432999) (end 155.028201 132.058801) (width 0.75) (layer B.Cu) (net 1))
 (segment (start 155.028201 132.058801) (end 155.7782 132.8088) (width 0.75) (layer B.Cu) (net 1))
 (segment (start 153.924 118.89232) (end 153.924 120.7008) (width 0.75) (layer B.Cu) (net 1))
 (segment (start 153.924 120.7008) (end 155.7274 122.5042) (width 0.75) (layer B.Cu) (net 1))
 (segment (start 153.82748 118.7958) (end 153.924 118.89232) (width 0.4) (layer F.Cu) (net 1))
 (segment (start 133.3158 112.268) (end 134.03199 112.268) (width 0.4) (layer F.Cu) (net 16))
 (segment (start 134.03199 112.268) (end 139.8016 106.49839) (width 0.4) (layer F.Cu) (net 16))
 (segment (start 139.8016 106.49839) (end 139.8016 106.2482) (width 0.4) (layer F.Cu) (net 16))
 (segment (start 140.969574 108.09784) (end 141.569574 107.49784) (width 0.4) (layer F.Cu) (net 17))
 (segment (start 139.899233 108.097841) (end 140.969574 108.09784) (width 0.4) (layer F.Cu) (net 17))
 (segment (start 134.429074 113.568) (end 139.899233 108.097841) (width 0.4) (layer F.Cu) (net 17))
 (segment (start 133.3158 113.568) (end 134.429074 113.568) (width 0.4) (layer F.Cu) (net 17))
 (segment (start 141.569574 107.49784) (end 142.217105 107.49784) (width 0.4) (layer F.Cu) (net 17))
 (segment (start 142.217105 107.49784) (end 143.466745 106.2482) (width 0.4) (layer F.Cu) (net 17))
 (segment (start 143.466745 106.2482) (end 143.80464 106.2482) (width 0.4) (layer F.Cu) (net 17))
 (segment (start 134.230531 112.918) (end 139.6507 107.497831) (width 0.4) (layer F.Cu) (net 18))
 (segment (start 133.3158 112.918) (end 134.230531 112.918) (width 0.4) (layer F.Cu) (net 18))
 (segment (start 139.6507 107.497831) (end 140.721041 107.497831) (width 0.4) (layer F.Cu) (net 18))
 (segment (start 140.721041 107.497831) (end 141.80312 106.415752) (width 0.4) (layer F.Cu) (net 18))
 (segment (start 141.80312 106.415752) (end 141.80312 106.2482) (width 0.4) (layer F.Cu) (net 18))
 (segment (start 141.818105 108.097851) (end 142.465637 108.097851) (width 0.4) (layer F.Cu) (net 19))
 (segment (start 143.2306 107.6452) (end 144.65681 107.6452) (width 0.4) (layer F.Cu) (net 19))
 (segment (start 142.8242 108.0516) (end 143.2306 107.6452) (width 0.4) (layer F.Cu) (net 19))
 (segment (start 134.627616 114.218) (end 140.147766 108.69785) (width 0.4) (layer F.Cu) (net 19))
 (segment (start 133.3158 114.218) (end 134.627616 114.218) (width 0.4) (layer F.Cu) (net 19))
 (segment (start 141.218107 108.697849) (end 141.818105 108.097851) (width 0.4) (layer F.Cu) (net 19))
 (segment (start 140.147766 108.69785) (end 141.218107 108.697849) (width 0.4) (layer F.Cu) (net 19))
 (segment (start 142.465637 108.097851) (end 142.511888 108.0516) (width 0.4) (layer F.Cu) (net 19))
 (segment (start 142.511888 108.0516) (end 142.8242 108.0516) (width 0.4) (layer F.Cu) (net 19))
 (segment (start 144.65681 107.6452) (end 145.80362 106.49839) (width 0.4) (layer F.Cu) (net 19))
 (segment (start 145.80362 106.49839) (end 145.80362 106.2482) (width 0.4) (layer F.Cu) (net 19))
 (segment (start 145.502199 114.228401) (end 144.826199 113.552401) (width 0.4) (layer F.Cu) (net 20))
 (segment (start 155.7274 130.1242) (end 154.577399 128.974199) (width 0.4) (layer F.Cu) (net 20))
 (segment (start 144.826199 113.552401) (end 144.826199 112.417967) (width 0.4) (layer F.Cu) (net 20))
 (segment (start 144.826199 112.417967) (end 144.676232 112.268) (width 0.4) (layer F.Cu) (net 20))
 (segment (start 147.491832 114.228401) (end 145.502199 114.228401) (width 0.4) (layer F.Cu) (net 20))
 (segment (start 149.226234 116.784806) (end 149.226234 115.962803) (width 0.4) (layer F.Cu) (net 20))
 (segment (start 154.577399 122.135971) (end 149.226234 116.784806) (width 0.4) (layer F.Cu) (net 20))
 (segment (start 144.676232 112.268) (end 140.0158 112.268) (width 0.4) (layer F.Cu) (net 20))
 (segment (start 140.0158 112.268) (end 139.1158 112.268) (width 0.4) (layer F.Cu) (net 20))
 (segment (start 149.226234 115.962803) (end 147.491832 114.228401) (width 0.4) (layer F.Cu) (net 20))
 (segment (start 154.577399 128.974199) (end 154.577399 122.135971) (width 0.4) (layer F.Cu) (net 20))
 (segment (start 147.2433 114.828412) (end 148.626223 116.211335) (width 0.4) (layer F.Cu) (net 21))
 (segment (start 144.226188 113.017978) (end 144.226188 113.800933) (width 0.4) (layer F.Cu) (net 21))
 (segment (start 155.028201 139.678801) (end 155.7782 140.4288) (width 0.4) (layer F.Cu) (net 21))
 (segment (start 153.977388 138.627988) (end 155.028201 139.678801) (width 0.4) (layer F.Cu) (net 21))
 (segment (start 144.226188 113.800933) (end 145.253667 114.828412) (width 0.4) (layer F.Cu) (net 21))
 (segment (start 148.626223 116.211335) (end 148.626223 117.033338) (width 0.4) (layer F.Cu) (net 21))
 (segment (start 148.626223 117.033338) (end 153.977388 122.384503) (width 0.4) (layer F.Cu) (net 21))
 (segment (start 153.977388 122.384503) (end 153.977388 138.627988) (width 0.4) (layer F.Cu) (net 21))
 (segment (start 144.12621 112.918) (end 144.226188 113.017978) (width 0.4) (layer F.Cu) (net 21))
 (segment (start 139.1158 112.918) (end 144.12621 112.918) (width 0.4) (layer F.Cu) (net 21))
 (segment (start 145.253667 114.828412) (end 147.2433 114.828412) (width 0.4) (layer F.Cu) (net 21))
 (segment (start 155.028201 150.253001) (end 155.7782 151.003) (width 0.4) (layer F.Cu) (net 4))
 (segment (start 153.377377 148.602177) (end 155.028201 150.253001) (width 0.4) (layer F.Cu) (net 4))
 (segment (start 148.026212 117.28187) (end 153.377377 122.633035) (width 0.4) (layer F.Cu) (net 4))
 (segment (start 148.026212 116.459867) (end 148.026212 117.28187) (width 0.4) (layer F.Cu) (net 4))
 (segment (start 143.626177 114.049465) (end 145.005135 115.428423) (width 0.4) (layer F.Cu) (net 4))
 (segment (start 153.377377 122.633035) (end 153.377377 148.602177) (width 0.4) (layer F.Cu) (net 4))
 (segment (start 139.1158 113.568) (end 143.576188 113.568) (width 0.4) (layer F.Cu) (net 4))
 (segment (start 146.994768 115.428423) (end 148.026212 116.459867) (width 0.4) (layer F.Cu) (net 4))
 (segment (start 145.005135 115.428423) (end 146.994768 115.428423) (width 0.4) (layer F.Cu) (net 4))
 (segment (start 143.576188 113.568) (end 143.626177 113.617989) (width 0.4) (layer F.Cu) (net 4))
 (segment (start 143.626177 113.617989) (end 143.626177 114.049465) (width 0.4) (layer F.Cu) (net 4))
 (segment (start 155.829 161.4932) (end 152.777366 158.441566) (width 0.4) (layer F.Cu) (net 22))
 (segment (start 152.777366 122.881566) (end 147.426201 117.530401) (width 0.4) (layer F.Cu) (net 22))
 (segment (start 152.777366 158.441566) (end 152.777366 122.881566) (width 0.4) (layer F.Cu) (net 22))
 (segment (start 143.026166 114.218) (end 139.1158 114.218) (width 0.4) (layer F.Cu) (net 22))
 (segment (start 147.426201 117.530401) (end 147.426201 116.708399) (width 0.4) (layer F.Cu) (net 22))
 (segment (start 147.426201 116.708399) (end 146.746236 116.028434) (width 0.4) (layer F.Cu) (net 22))
 (segment (start 146.746236 116.028434) (end 144.756603 116.028434) (width 0.4) (layer F.Cu) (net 22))
 (segment (start 144.756603 116.028434) (end 143.026166 114.297997) (width 0.4) (layer F.Cu) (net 22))
 (segment (start 143.026166 114.297997) (end 143.026166 114.218) (width 0.4) (layer F.Cu) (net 22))
 (segment (start 145.4912 165.5826) (end 145.4912 167.18223) (width 0.75) (layer B.Cu) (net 9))
 (segment (start 132.103169 161.094681) (end 132.103169 158.975799) (width 0.75) (layer B.Cu) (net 9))
 (segment (start 145.4912 167.18223) (end 145.279752 167.393678) (width 0.75) (layer B.Cu) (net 9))
 (segment (start 145.279752 167.393678) (end 139.250478 167.393678) (width 0.75) (layer B.Cu) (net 9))
 (segment (start 138.3538 166.497) (end 138.3538 165.274998) (width 0.75) (layer B.Cu) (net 9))
 (segment (start 138.3538 165.274998) (end 134.419602 161.3408) (width 0.75) (layer B.Cu) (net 9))
 (segment (start 139.250478 167.393678) (end 138.3538 166.497) (width 0.75) (layer B.Cu) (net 9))
 (segment (start 134.419602 161.3408) (end 132.349288 161.3408) (width 0.75) (layer B.Cu) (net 9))
 (segment (start 132.349288 161.3408) (end 132.103169 161.094681) (width 0.75) (layer B.Cu) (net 9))
 (segment (start 132.103169 158.975799) (end 133.045248 158.03372) (width 0.75) (layer B.Cu) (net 9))
 (segment (start 133.045248 158.03372) (end 133.5278 158.03372) (width 0.75) (layer B.Cu) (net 9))
 (segment (start 133.6294 136.58088) (end 133.37921 136.58088) (width 0.75) (layer B.Cu) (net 9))
 (segment (start 133.37921 136.58088) (end 132.153969 135.355639) (width 0.75) (layer B.Cu) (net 9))
 (segment (start 132.153969 135.355639) (end 132.153969 127.235959) (width 0.75) (layer B.Cu) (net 9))
 (segment (start 132.153969 127.235959) (end 133.096048 126.29388) (width 0.75) (layer B.Cu) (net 9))
 (segment (start 133.096048 126.29388) (end 133.5786 126.29388) (width 0.75) (layer B.Cu) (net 9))
 (segment (start 133.6548 147.50288) (end 133.40461 147.50288) (width 0.75) (layer B.Cu) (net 9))
 (segment (start 133.40461 147.50288) (end 132.204769 146.303039) (width 0.75) (layer B.Cu) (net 9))
 (segment (start 132.204769 146.303039) (end 132.204769 137.522959) (width 0.75) (layer B.Cu) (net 9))
 (segment (start 132.204769 137.522959) (end 133.146848 136.58088) (width 0.75) (layer B.Cu) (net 9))
 (segment (start 133.146848 136.58088) (end 133.6294 136.58088) (width 0.75) (layer B.Cu) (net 9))
 (segment (start 133.5278 158.03372) (end 133.27761 158.03372) (width 0.75) (layer B.Cu) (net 9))
 (segment (start 132.10316 156.85927) (end 132.10316 148.571968) (width 0.75) (layer B.Cu) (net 9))
 (segment (start 133.27761 158.03372) (end 132.10316 156.85927) (width 0.75) (layer B.Cu) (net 9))
 (segment (start 132.10316 148.571968) (end 133.172248 147.50288) (width 0.75) (layer B.Cu) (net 9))
 (segment (start 133.172248 147.50288) (end 133.6548 147.50288) (width 0.75) (layer B.Cu) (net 9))
 (segment (start 150.095649 113.214849) (end 150.8674 113.214849) (width 0.4) (layer B.Cu) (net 2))
 (segment (start 150.8674 113.214849) (end 151.291664 113.214849) (width 0.4) (layer B.Cu) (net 2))
 (segment (start 150.0886 113.2078) (end 150.095649 113.214849) (width 0.4) (layer B.Cu) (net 2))
 (segment (start 151.298713 113.2078) (end 151.291664 113.214849) (width 0.4) (layer F.Cu) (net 2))
 (segment (start 152.48128 113.2078) (end 151.298713 113.2078) (width 0.4) (layer F.Cu) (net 2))
 (via (at 151.291664 113.214849) (size 0.6) (drill 0.4) (layers F.Cu B.Cu) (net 2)))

